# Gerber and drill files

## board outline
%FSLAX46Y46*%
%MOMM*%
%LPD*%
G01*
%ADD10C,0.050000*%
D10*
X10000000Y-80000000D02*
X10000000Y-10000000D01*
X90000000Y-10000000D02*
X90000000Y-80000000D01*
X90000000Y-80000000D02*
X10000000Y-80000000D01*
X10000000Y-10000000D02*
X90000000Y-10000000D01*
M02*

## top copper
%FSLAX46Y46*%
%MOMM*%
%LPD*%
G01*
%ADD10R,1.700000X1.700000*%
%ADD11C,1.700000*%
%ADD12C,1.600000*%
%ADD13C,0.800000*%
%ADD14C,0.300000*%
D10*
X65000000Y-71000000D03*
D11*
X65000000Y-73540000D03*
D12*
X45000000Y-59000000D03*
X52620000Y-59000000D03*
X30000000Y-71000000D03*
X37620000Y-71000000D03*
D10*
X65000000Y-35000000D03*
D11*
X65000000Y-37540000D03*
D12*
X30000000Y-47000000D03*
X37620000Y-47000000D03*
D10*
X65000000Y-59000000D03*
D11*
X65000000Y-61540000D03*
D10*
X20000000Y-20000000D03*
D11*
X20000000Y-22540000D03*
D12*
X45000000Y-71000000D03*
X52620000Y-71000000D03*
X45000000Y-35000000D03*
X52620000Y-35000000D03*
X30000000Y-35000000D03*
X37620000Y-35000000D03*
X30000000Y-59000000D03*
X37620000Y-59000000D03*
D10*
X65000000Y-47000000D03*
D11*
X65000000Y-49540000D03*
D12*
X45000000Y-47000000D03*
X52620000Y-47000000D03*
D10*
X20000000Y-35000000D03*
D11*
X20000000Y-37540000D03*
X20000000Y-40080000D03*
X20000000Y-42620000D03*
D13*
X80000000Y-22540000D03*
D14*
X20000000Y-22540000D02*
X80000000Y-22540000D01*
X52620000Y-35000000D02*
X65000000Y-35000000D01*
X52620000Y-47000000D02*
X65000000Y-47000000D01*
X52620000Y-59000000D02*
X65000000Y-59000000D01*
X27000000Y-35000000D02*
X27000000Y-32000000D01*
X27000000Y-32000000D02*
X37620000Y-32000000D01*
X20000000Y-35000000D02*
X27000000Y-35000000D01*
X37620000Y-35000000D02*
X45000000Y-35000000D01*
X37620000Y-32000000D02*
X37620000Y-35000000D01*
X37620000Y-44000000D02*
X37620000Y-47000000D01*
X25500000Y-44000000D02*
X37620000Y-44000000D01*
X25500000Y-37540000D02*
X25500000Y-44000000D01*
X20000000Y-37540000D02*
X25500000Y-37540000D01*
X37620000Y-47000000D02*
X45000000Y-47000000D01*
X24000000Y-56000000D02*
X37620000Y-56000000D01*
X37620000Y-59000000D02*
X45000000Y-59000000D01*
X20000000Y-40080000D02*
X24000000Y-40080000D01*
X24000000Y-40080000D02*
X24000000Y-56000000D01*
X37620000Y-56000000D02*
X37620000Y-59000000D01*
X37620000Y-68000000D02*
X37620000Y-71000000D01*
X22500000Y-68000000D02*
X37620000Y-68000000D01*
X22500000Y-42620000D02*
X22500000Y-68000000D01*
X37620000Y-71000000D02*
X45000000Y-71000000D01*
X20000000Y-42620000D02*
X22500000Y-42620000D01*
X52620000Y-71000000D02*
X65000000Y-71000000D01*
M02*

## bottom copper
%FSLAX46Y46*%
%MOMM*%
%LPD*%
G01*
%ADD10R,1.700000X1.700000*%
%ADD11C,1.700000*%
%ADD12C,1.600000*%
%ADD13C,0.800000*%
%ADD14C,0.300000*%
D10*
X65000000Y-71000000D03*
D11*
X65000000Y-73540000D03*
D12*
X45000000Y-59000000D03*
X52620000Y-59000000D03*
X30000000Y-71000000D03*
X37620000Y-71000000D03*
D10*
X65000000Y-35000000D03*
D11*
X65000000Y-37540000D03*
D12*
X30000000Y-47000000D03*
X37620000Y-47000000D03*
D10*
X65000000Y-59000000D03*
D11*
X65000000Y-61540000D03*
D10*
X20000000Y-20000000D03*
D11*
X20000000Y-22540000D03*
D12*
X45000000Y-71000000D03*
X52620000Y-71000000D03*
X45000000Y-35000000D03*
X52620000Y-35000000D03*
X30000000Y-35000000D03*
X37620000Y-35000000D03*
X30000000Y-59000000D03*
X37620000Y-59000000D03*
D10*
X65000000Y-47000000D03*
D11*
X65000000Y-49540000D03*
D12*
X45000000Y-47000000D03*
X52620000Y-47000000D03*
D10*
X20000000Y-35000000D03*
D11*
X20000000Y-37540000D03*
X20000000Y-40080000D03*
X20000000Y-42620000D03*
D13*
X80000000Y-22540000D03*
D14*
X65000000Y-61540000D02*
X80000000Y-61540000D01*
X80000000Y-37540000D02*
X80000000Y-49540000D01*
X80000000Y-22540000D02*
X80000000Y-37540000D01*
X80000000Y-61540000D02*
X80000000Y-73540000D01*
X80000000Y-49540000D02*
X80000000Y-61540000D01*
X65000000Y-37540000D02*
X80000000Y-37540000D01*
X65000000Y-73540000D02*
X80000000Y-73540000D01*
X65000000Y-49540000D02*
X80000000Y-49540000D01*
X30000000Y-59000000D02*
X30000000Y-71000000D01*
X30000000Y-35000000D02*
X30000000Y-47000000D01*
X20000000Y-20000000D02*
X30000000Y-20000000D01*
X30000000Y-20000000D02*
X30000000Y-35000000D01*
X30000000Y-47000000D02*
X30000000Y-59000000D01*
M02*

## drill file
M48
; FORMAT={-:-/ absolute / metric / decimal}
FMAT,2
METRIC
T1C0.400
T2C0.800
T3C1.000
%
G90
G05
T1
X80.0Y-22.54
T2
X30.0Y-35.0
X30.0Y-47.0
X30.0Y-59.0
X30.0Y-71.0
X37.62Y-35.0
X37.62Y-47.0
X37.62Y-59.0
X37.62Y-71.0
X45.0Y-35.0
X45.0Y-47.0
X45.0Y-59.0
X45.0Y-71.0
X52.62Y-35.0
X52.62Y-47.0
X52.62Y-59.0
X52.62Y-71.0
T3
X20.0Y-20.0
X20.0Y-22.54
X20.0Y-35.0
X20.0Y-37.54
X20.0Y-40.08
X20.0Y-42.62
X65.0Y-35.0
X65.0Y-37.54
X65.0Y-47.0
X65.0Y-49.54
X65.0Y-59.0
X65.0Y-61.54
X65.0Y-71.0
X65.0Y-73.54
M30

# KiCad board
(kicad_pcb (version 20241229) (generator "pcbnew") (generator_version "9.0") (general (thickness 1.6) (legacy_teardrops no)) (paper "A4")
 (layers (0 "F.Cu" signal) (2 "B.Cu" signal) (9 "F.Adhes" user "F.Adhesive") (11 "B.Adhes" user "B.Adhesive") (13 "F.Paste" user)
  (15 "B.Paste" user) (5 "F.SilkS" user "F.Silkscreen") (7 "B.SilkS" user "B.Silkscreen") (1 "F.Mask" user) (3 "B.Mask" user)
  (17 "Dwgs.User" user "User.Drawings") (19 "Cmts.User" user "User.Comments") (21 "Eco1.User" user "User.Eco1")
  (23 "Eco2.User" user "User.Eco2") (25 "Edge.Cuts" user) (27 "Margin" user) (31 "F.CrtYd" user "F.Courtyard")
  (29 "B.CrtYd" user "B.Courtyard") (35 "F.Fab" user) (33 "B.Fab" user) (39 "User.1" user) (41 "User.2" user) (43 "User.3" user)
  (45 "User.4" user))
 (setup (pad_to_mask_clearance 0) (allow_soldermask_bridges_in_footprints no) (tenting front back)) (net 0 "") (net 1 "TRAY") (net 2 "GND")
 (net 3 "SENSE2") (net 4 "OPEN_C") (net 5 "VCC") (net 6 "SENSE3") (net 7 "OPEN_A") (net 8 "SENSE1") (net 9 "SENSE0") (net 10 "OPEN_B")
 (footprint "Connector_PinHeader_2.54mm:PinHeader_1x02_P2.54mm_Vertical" (layer "F.Cu") (at 65 71)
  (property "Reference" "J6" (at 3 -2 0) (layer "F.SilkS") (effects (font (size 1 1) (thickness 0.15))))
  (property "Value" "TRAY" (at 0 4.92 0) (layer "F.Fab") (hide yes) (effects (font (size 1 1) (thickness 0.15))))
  (pad "1" thru_hole rect (at 0 0) (size 1.7 1.7) (drill 1) (layers "*.Cu" "*.Mask") (remove_unused_layers no) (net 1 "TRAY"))
  (pad "2" thru_hole circle (at 0 2.54) (size 1.7 1.7) (drill 1) (layers "*.Cu" "*.Mask") (remove_unused_layers no) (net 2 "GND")))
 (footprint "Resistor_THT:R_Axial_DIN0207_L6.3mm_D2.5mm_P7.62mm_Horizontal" (layer "F.Cu") (at 45 59)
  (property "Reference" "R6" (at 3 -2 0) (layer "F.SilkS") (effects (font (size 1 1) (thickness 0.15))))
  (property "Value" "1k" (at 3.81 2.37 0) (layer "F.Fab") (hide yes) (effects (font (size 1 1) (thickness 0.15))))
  (pad "1" thru_hole circle (at 0 0) (size 1.6 1.6) (drill 0.8) (layers "*.Cu" "*.Mask") (remove_unused_layers no) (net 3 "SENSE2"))
  (pad "2" thru_hole circle (at 7.62 0) (size 1.6 1.6) (drill 0.8) (layers "*.Cu" "*.Mask") (remove_unused_layers no) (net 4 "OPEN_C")))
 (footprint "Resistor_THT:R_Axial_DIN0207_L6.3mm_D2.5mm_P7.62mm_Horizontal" (layer "F.Cu") (at 30 71)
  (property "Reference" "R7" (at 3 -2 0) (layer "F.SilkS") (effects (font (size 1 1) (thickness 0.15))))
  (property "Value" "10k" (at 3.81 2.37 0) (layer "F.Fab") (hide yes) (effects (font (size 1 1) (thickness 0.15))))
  (pad "1" thru_hole circle (at 0 0) (size 1.6 1.6) (drill 0.8) (layers "*.Cu" "*.Mask") (remove_unused_layers no) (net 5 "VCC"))
  (pad "2" thru_hole circle (at 7.62 0) (size 1.6 1.6) (drill 0.8) (layers "*.Cu" "*.Mask") (remove_unused_layers no) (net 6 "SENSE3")))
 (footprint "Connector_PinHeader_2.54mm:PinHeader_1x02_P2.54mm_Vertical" (layer "F.Cu") (at 65 35)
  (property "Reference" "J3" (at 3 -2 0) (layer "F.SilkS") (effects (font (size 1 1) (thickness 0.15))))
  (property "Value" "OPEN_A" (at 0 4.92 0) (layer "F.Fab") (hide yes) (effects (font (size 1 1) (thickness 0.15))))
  (pad "1" thru_hole rect (at 0 0) (size 1.7 1.7) (drill 1) (layers "*.Cu" "*.Mask") (remove_unused_layers no) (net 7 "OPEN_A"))
  (pad "2" thru_hole circle (at 0 2.54) (size 1.7 1.7) (drill 1) (layers "*.Cu" "*.Mask") (remove_unused_layers no) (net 2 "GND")))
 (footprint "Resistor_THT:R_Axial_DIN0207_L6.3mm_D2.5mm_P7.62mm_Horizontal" (layer "F.Cu") (at 30 47)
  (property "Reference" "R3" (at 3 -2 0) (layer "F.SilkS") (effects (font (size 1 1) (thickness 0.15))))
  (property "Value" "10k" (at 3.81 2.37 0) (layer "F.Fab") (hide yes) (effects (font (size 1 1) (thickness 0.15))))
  (pad "1" thru_hole circle (at 0 0) (size 1.6 1.6) (drill 0.8) (layers "*.Cu" "*.Mask") (remove_unused_layers no) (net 5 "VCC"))
  (pad "2" thru_hole circle (at 7.62 0) (size 1.6 1.6) (drill 0.8) (layers "*.Cu" "*.Mask") (remove_unused_layers no) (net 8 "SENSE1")))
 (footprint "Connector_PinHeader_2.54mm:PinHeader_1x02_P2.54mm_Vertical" (layer "F.Cu") (at 65 59)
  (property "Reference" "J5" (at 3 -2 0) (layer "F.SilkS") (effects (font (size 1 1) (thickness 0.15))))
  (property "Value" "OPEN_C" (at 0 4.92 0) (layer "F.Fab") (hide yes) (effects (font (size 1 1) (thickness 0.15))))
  (pad "1" thru_hole rect (at 0 0) (size 1.7 1.7) (drill 1) (layers "*.Cu" "*.Mask") (remove_unused_layers no) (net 4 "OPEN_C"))
  (pad "2" thru_hole circle (at 0 2.54) (size 1.7 1.7) (drill 1) (layers "*.Cu" "*.Mask") (remove_unused_layers no) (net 2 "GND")))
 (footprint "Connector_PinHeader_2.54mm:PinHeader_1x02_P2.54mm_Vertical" (layer "F.Cu") (at 20 20)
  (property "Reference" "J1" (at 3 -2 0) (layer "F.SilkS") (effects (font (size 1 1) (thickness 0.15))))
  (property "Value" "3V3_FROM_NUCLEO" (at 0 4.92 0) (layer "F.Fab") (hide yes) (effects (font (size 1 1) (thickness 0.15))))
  (pad "1" thru_hole rect (at 0 0) (size 1.7 1.7) (drill 1) (layers "*.Cu" "*.Mask") (remove_unused_layers no) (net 5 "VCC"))
  (pad "2" thru_hole circle (at 0 2.54) (size 1.7 1.7) (drill 1) (layers "*.Cu" "*.Mask") (remove_unused_layers no) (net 2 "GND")))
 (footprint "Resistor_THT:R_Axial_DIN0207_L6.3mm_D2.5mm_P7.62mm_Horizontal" (layer "F.Cu") (at 45 71)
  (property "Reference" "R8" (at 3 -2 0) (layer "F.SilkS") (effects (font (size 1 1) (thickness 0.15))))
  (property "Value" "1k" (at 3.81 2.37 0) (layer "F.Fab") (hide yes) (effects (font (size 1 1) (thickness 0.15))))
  (pad "1" thru_hole circle (at 0 0) (size 1.6 1.6) (drill 0.8) (layers "*.Cu" "*.Mask") (remove_unused_layers no) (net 6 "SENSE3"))
  (pad "2" thru_hole circle (at 7.62 0) (size 1.6 1.6) (drill 0.8) (layers "*.Cu" "*.Mask") (remove_unused_layers no) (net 1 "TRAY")))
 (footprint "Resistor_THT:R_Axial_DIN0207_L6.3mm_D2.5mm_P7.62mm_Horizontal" (layer "F.Cu") (at 45 35)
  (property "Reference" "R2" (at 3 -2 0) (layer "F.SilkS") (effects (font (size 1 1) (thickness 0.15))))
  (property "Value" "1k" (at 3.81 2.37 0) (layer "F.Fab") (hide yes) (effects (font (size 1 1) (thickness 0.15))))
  (pad "1" thru_hole circle (at 0 0) (size 1.6 1.6) (drill 0.8) (layers "*.Cu" "*.Mask") (remove_unused_layers no) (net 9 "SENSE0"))
  (pad "2" thru_hole circle (at 7.62 0) (size 1.6 1.6) (drill 0.8) (layers "*.Cu" "*.Mask") (remove_unused_layers no) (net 7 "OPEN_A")))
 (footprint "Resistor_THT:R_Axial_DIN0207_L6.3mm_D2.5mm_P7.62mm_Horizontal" (layer "F.Cu") (at 30 35)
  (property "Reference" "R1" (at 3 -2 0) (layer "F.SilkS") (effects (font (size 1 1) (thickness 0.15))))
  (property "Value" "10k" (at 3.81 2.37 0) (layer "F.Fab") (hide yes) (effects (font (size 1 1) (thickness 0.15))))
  (pad "1" thru_hole circle (at 0 0) (size 1.6 1.6) (drill 0.8) (layers "*.Cu" "*.Mask") (remove_unused_layers no) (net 5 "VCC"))
  (pad "2" thru_hole circle (at 7.62 0) (size 1.6 1.6) (drill 0.8) (layers "*.Cu" "*.Mask") (remove_unused_layers no) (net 9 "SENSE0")))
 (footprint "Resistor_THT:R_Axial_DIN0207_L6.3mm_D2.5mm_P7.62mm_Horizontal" (layer "F.Cu") (at 30 59)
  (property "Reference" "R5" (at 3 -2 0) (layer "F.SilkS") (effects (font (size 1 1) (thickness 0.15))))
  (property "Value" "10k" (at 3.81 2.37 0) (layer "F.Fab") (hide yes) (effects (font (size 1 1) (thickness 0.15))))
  (pad "1" thru_hole circle (at 0 0) (size 1.6 1.6) (drill 0.8) (layers "*.Cu" "*.Mask") (remove_unused_layers no) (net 5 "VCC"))
  (pad "2" thru_hole circle (at 7.62 0) (size 1.6 1.6) (drill 0.8) (layers "*.Cu" "*.Mask") (remove_unused_layers no) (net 3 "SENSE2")))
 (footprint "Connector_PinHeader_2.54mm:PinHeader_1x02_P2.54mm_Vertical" (layer "F.Cu") (at 65 47)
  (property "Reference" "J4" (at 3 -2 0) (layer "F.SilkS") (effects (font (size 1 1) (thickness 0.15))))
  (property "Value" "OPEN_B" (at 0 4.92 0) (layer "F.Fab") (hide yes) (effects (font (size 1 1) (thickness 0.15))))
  (pad "1" thru_hole rect (at 0 0) (size 1.7 1.7) (drill 1) (layers "*.Cu" "*.Mask") (remove_unused_layers no) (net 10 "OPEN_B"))
  (pad "2" thru_hole circle (at 0 2.54) (size 1.7 1.7) (drill 1) (layers "*.Cu" "*.Mask") (remove_unused_layers no) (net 2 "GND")))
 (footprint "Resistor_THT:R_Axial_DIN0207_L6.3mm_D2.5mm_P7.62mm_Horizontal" (layer "F.Cu") (at 45 47)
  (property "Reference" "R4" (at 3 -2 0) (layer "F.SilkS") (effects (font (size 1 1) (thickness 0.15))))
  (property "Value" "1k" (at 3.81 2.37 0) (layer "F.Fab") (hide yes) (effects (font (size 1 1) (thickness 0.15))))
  (pad "1" thru_hole circle (at 0 0) (size 1.6 1.6) (drill 0.8) (layers "*.Cu" "*.Mask") (remove_unused_layers no) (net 8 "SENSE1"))
  (pad "2" thru_hole circle (at 7.62 0) (size 1.6 1.6) (drill 0.8) (layers "*.Cu" "*.Mask") (remove_unused_layers no) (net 10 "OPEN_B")))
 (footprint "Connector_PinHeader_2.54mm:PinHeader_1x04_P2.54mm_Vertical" (layer "F.Cu") (at 20 35)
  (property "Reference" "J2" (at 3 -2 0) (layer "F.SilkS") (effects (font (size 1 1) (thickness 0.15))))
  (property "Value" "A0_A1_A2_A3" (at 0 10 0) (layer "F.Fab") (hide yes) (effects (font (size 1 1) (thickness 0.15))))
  (pad "1" thru_hole rect (at 0 0) (size 1.7 1.7) (drill 1) (layers "*.Cu" "*.Mask") (remove_unused_layers no) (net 9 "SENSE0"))
  (pad "2" thru_hole circle (at 0 2.54) (size 1.7 1.7) (drill 1) (layers "*.Cu" "*.Mask") (remove_unused_layers no) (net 8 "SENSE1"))
  (pad "3" thru_hole circle (at 0 5.08) (size 1.7 1.7) (drill 1) (layers "*.Cu" "*.Mask") (remove_unused_layers no) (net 3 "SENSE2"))
  (pad "4" thru_hole circle (at 0 7.62) (size 1.7 1.7) (drill 1) (layers "*.Cu" "*.Mask") (remove_unused_layers no) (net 6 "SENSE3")))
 (gr_line (start 10 80) (end 10 10) (stroke (width 0.05) (type default)) (layer "Edge.Cuts"))
 (gr_line (start 90 10) (end 90 80) (stroke (width 0.05) (type default)) (layer "Edge.Cuts"))
 (gr_line (start 90 80) (end 10 80) (stroke (width 0.05) (type default)) (layer "Edge.Cuts"))
 (gr_line (start 10 10) (end 90 10) (stroke (width 0.05) (type default)) (layer "Edge.Cuts"))
 (segment (start 20 22.54) (end 80 22.54) (width 0.3) (layer "F.Cu") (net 2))
 (via (at 80 22.54) (size 0.8) (drill 0.4) (layers "F.Cu" "B.Cu") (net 2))
 (segment (start 65 61.54) (end 80 61.54) (width 0.3) (layer "B.Cu") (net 2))
 (segment (start 80 37.54) (end 80 49.54) (width 0.3) (layer "B.Cu") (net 2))
 (segment (start 80 22.54) (end 80 37.54) (width 0.3) (layer "B.Cu") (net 2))
 (segment (start 80 61.54) (end 80 73.54) (width 0.3) (layer "B.Cu") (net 2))
 (segment (start 80 49.54) (end 80 61.54) (width 0.3) (layer "B.Cu") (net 2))
 (segment (start 65 37.54) (end 80 37.54) (width 0.3) (layer "B.Cu") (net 2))
 (segment (start 65 73.54) (end 80 73.54) (width 0.3) (layer "B.Cu") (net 2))
 (segment (start 65 49.54) (end 80 49.54) (width 0.3) (layer "B.Cu") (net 2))
 (segment (start 52.62 35) (end 65 35) (width 0.3) (layer "F.Cu") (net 7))
 (segment (start 52.62 47) (end 65 47) (width 0.3) (layer "F.Cu") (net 10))
 (segment (start 52.62 59) (end 65 59) (width 0.3) (layer "F.Cu") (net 4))
 (segment (start 27 35) (end 27 32) (width 0.3) (layer "F.Cu") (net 9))
 (segment (start 27 32) (end 37.62 32) (width 0.3) (layer "F.Cu") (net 9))
 (segment (start 20 35) (end 27 35) (width 0.3) (layer "F.Cu") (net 9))
 (segment (start 37.62 35) (end 45 35) (width 0.3) (layer "F.Cu") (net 9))
 (segment (start 37.62 32) (end 37.62 35) (width 0.3) (layer "F.Cu") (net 9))
 (segment (start 37.62 44) (end 37.62 47) (width 0.3) (layer "F.Cu") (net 8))
 (segment (start 25.5 44) (end 37.62 44) (width 0.3) (layer "F.Cu") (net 8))
 (segment (start 25.5 37.54) (end 25.5 44) (width 0.3) (layer "F.Cu") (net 8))
 (segment (start 20 37.54) (end 25.5 37.54) (width 0.3) (layer "F.Cu") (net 8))
 (segment (start 37.62 47) (end 45 47) (width 0.3) (layer "F.Cu") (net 8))
 (segment (start 24 56) (end 37.62 56) (width 0.3) (layer "F.Cu") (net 3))
 (segment (start 37.62 59) (end 45 59) (width 0.3) (layer "F.Cu") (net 3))
 (segment (start 20 40.08) (end 24 40.08) (width 0.3) (layer "F.Cu") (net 3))
 (segment (start 24 40.08) (end 24 56) (width 0.3) (layer "F.Cu") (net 3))
 (segment (start 37.62 56) (end 37.62 59) (width 0.3) (layer "F.Cu") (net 3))
 (segment (start 37.62 68) (end 37.62 71) (width 0.3) (layer "F.Cu") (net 6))
 (segment (start 22.5 68) (end 37.62 68) (width 0.3) (layer "F.Cu") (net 6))
 (segment (start 22.5 42.62) (end 22.5 68) (width 0.3) (layer "F.Cu") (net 6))
 (segment (start 37.62 71) (end 45 71) (width 0.3) (layer "F.Cu") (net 6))
 (segment (start 20 42.62) (end 22.5 42.62) (width 0.3) (layer "F.Cu") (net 6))
 (segment (start 52.62 71) (end 65 71) (width 0.3) (layer "F.Cu") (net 1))
 (segment (start 30 59) (end 30 71) (width 0.3) (layer "B.Cu") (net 5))
 (segment (start 30 35) (end 30 47) (width 0.3) (layer "B.Cu") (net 5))
 (segment (start 20 20) (end 30 20) (width 0.3) (layer "B.Cu") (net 5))
 (segment (start 30 20) (end 30 35) (width 0.3) (layer "B.Cu") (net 5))
 (segment (start 30 47) (end 30 59) (width 0.3) (layer "B.Cu") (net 5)))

